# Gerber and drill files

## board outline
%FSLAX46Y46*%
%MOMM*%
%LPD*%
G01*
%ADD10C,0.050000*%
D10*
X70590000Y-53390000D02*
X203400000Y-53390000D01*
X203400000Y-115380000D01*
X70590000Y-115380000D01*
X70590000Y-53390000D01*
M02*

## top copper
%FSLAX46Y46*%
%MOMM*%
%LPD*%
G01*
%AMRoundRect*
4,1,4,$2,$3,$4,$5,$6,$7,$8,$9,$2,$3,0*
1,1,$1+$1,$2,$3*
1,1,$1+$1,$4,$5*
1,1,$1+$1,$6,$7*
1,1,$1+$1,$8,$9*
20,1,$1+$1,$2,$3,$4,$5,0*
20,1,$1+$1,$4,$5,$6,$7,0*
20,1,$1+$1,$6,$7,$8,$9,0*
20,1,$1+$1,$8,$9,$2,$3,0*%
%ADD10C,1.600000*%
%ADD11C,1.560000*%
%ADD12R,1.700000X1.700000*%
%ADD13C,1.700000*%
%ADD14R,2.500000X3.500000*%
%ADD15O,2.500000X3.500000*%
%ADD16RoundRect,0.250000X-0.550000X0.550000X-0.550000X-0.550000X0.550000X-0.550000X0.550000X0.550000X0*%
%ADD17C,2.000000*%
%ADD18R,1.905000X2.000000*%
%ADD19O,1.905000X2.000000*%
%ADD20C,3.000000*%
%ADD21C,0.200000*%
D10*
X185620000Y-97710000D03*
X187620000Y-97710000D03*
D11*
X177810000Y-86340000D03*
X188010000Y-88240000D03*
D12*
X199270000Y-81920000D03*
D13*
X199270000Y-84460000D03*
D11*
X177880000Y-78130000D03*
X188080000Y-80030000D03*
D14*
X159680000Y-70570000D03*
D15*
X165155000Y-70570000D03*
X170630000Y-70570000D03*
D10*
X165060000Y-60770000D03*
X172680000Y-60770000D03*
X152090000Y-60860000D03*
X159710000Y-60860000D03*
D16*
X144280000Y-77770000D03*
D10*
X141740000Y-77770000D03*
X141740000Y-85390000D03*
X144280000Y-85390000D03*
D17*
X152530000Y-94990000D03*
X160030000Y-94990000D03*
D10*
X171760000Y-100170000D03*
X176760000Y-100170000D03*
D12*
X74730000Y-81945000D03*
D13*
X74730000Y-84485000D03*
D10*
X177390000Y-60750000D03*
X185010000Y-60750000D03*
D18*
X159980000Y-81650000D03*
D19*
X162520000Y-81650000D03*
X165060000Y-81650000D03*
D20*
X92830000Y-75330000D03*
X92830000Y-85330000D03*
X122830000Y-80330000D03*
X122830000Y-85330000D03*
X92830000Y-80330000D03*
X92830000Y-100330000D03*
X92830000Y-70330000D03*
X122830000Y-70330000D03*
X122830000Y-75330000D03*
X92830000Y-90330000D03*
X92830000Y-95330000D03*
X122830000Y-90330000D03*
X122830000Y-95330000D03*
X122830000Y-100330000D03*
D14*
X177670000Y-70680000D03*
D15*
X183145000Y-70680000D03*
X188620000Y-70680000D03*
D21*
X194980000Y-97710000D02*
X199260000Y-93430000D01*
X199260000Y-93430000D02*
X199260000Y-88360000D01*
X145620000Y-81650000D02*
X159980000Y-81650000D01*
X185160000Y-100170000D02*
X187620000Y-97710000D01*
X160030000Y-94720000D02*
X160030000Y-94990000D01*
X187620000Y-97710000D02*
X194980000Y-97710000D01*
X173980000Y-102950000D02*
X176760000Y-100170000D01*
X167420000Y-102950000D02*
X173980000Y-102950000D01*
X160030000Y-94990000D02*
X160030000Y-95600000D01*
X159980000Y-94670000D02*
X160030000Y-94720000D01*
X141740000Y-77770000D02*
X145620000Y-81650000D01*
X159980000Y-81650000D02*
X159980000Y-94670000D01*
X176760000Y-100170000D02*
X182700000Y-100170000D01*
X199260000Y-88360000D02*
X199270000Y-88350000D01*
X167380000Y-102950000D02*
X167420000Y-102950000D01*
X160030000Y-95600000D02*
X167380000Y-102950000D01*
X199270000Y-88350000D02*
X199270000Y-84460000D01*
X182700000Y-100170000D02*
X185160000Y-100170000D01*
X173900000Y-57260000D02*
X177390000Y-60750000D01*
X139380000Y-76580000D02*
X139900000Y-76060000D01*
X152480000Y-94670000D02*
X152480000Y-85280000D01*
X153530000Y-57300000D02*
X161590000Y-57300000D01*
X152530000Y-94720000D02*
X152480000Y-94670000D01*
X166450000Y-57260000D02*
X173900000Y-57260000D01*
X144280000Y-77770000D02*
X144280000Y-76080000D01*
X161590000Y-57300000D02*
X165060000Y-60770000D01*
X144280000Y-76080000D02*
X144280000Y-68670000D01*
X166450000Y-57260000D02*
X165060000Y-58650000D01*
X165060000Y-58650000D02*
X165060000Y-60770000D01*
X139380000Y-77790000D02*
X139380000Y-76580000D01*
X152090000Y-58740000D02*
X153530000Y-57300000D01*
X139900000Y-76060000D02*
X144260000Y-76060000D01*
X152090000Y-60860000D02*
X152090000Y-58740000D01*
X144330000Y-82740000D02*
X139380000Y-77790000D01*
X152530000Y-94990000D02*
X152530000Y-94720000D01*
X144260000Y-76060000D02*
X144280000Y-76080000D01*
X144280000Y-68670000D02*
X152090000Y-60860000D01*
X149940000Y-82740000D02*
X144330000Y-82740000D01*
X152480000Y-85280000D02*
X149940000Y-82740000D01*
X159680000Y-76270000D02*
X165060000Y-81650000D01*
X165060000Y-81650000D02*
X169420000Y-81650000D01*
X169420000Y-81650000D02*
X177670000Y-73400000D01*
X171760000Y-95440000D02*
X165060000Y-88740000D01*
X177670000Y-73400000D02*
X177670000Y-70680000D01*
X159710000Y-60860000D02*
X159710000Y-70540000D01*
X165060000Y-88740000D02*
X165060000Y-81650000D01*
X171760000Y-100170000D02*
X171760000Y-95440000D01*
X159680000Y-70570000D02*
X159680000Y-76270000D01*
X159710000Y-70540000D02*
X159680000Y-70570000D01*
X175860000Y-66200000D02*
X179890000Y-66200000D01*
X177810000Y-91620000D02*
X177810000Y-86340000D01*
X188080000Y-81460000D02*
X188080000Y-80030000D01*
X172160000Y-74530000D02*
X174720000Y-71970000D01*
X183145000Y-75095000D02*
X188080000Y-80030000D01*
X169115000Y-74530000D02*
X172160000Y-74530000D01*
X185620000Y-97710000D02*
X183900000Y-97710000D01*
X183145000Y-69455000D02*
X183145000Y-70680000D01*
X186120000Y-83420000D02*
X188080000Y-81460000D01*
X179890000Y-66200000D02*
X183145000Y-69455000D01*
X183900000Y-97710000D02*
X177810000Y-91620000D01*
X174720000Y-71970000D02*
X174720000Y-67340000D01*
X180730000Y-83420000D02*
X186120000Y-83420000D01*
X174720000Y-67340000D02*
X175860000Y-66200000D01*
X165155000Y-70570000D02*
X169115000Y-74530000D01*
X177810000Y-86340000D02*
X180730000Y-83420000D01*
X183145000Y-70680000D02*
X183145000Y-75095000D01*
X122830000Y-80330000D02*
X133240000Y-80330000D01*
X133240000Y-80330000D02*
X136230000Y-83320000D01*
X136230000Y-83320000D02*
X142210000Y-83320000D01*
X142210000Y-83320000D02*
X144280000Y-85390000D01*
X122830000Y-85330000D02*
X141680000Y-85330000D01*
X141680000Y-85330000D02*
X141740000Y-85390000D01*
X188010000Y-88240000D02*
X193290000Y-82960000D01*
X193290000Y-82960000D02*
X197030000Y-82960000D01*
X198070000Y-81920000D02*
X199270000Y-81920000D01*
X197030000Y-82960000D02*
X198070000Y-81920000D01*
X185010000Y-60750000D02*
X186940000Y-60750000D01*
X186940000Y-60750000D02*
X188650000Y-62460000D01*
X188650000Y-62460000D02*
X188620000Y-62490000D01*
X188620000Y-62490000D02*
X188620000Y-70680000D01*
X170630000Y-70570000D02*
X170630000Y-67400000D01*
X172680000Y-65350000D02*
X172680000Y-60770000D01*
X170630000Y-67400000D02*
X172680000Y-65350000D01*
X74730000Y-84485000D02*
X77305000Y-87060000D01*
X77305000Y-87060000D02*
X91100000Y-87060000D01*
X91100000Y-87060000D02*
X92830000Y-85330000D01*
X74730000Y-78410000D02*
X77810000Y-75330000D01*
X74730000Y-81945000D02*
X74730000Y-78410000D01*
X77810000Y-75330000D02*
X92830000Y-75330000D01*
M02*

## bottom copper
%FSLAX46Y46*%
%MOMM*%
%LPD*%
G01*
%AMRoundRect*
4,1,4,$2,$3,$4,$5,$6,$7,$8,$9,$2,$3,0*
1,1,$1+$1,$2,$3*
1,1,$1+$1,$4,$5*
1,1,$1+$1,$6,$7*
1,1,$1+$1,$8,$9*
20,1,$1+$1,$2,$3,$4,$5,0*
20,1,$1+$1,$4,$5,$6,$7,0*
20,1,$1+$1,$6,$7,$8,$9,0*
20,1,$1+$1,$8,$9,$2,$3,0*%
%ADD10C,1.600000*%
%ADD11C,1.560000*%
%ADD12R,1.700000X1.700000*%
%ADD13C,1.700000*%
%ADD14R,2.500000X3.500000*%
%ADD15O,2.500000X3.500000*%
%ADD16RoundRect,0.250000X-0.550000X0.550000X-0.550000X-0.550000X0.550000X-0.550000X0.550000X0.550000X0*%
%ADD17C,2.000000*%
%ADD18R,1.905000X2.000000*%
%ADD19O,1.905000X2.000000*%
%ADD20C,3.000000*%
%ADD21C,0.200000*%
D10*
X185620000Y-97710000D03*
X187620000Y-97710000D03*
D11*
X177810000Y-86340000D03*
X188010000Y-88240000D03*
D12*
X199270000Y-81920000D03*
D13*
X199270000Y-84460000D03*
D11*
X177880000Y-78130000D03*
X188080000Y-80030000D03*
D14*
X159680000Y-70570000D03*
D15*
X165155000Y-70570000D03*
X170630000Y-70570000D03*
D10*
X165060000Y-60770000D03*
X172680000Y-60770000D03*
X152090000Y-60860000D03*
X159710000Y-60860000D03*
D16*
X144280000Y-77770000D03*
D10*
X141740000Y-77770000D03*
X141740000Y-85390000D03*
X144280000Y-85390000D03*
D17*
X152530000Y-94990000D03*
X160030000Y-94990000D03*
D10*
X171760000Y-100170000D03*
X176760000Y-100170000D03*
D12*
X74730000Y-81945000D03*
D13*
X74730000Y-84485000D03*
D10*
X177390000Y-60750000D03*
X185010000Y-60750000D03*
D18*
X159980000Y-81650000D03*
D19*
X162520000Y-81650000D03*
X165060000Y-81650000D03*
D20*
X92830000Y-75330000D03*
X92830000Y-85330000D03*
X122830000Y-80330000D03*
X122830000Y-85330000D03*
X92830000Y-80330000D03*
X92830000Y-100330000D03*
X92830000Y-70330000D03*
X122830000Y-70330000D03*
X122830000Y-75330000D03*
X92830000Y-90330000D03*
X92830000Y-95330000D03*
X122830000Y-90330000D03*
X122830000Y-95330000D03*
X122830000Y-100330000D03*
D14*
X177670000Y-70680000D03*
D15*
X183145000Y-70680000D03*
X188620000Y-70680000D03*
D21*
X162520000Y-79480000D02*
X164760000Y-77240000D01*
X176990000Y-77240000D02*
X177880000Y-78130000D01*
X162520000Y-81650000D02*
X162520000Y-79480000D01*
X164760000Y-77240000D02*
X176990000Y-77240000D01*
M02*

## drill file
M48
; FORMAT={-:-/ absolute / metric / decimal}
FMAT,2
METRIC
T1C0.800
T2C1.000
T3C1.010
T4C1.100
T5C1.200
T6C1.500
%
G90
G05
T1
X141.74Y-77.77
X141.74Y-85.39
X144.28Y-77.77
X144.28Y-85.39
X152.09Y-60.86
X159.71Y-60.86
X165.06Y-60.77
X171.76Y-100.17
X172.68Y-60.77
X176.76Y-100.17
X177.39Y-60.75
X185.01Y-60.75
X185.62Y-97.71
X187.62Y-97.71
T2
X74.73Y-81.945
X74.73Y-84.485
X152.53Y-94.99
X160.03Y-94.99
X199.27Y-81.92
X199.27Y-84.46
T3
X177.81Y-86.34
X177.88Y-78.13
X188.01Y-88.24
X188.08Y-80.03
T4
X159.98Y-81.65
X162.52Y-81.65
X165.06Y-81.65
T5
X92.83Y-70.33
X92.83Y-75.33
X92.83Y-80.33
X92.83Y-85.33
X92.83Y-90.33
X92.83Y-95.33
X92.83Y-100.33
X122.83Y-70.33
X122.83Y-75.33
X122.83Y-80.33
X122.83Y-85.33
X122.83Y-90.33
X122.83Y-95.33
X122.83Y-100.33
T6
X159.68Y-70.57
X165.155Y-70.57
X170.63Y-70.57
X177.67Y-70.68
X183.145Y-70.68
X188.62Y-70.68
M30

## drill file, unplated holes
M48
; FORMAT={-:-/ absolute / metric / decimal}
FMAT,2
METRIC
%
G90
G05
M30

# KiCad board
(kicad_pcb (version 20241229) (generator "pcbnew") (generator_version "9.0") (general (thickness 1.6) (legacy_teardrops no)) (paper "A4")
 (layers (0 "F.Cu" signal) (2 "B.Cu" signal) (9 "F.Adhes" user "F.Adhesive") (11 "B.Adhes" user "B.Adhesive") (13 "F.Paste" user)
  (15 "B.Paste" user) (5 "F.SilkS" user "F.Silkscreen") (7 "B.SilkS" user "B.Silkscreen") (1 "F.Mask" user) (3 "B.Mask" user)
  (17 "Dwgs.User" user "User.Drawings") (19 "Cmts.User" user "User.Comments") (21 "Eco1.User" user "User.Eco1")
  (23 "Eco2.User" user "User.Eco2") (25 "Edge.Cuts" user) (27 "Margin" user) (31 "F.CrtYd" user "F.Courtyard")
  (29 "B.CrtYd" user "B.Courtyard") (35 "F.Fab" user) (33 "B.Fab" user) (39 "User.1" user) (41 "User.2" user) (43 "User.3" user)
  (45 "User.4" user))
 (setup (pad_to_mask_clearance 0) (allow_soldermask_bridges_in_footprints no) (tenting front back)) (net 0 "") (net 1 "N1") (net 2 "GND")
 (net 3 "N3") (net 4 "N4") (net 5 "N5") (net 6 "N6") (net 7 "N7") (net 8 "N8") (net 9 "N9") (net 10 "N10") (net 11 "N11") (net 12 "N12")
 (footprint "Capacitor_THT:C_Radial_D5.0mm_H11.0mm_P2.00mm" (layer "F.Cu") (at 185.62 97.71)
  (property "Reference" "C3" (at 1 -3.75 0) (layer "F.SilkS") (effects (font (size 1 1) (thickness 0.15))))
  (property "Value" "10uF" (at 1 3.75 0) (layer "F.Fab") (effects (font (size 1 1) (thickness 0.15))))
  (pad "1" thru_hole circle (at 0 0) (size 1.6 1.6) (drill 0.8) (layers "*.Cu" "*.Mask") (remove_unused_layers no) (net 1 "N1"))
  (pad "2" thru_hole circle (at 2 0) (size 1.6 1.6) (drill 0.8) (layers "*.Cu" "*.Mask") (remove_unused_layers no) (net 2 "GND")))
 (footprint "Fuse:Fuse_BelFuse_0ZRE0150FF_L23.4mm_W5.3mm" (layer "F.Cu") (at 177.81 86.34)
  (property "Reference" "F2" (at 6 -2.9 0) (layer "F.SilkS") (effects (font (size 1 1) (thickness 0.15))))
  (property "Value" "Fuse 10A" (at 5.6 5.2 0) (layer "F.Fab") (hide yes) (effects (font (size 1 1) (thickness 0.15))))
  (pad "1" thru_hole circle (at 0 0) (size 1.56 1.56) (drill 1.01) (layers "*.Cu" "*.Mask") (remove_unused_layers no) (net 1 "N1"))
  (pad "2" thru_hole circle (at 10.2 1.9) (size 1.56 1.56) (drill 1.01) (layers "*.Cu" "*.Mask") (remove_unused_layers no) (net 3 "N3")))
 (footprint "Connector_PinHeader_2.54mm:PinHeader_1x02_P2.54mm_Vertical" (layer "F.Cu") (at 199.27 81.92)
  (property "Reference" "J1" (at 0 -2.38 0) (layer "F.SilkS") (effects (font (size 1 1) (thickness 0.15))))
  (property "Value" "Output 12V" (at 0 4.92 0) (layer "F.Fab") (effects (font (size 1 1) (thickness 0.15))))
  (pad "1" thru_hole rect (at 0 0) (size 1.7 1.7) (drill 1) (layers "*.Cu" "*.Mask") (remove_unused_layers no) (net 3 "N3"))
  (pad "2" thru_hole circle (at 0 2.54) (size 1.7 1.7) (drill 1) (layers "*.Cu" "*.Mask") (remove_unused_layers no) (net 2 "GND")))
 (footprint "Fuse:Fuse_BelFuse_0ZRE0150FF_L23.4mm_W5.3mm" (layer "F.Cu") (at 177.88 78.13)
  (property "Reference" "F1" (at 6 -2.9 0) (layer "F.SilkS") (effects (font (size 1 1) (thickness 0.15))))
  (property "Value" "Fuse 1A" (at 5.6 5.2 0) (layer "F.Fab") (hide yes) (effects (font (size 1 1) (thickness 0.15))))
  (pad "1" thru_hole circle (at 0 0) (size 1.56 1.56) (drill 1.01) (layers "*.Cu" "*.Mask") (remove_unused_layers no) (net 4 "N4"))
  (pad "2" thru_hole circle (at 10.2 1.9) (size 1.56 1.56) (drill 1.01) (layers "*.Cu" "*.Mask") (remove_unused_layers no) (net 1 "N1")))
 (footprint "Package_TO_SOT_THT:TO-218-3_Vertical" (layer "F.Cu") (at 159.68 70.57)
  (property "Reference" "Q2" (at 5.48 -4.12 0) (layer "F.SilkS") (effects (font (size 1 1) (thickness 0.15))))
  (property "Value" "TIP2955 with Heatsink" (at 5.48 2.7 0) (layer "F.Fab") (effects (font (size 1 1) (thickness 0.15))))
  (pad "1" thru_hole rect (at 0 0) (size 2.5 3.5) (drill 1.5) (layers "*.Cu" "*.Mask") (remove_unused_layers no) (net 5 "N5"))
  (pad "2" thru_hole oval (at 5.475 0) (size 2.5 3.5) (drill 1.5) (layers "*.Cu" "*.Mask") (remove_unused_layers no) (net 1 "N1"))
  (pad "3" thru_hole oval (at 10.95 0) (size 2.5 3.5) (drill 1.5) (layers "*.Cu" "*.Mask") (remove_unused_layers no) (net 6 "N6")))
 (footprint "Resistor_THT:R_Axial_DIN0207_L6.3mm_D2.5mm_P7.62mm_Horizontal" (layer "F.Cu") (at 165.06 60.77)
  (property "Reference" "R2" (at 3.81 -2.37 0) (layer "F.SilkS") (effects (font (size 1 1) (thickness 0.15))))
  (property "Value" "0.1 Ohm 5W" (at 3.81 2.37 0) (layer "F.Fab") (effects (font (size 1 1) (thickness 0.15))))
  (pad "1" thru_hole circle (at 0 0) (size 1.6 1.6) (drill 0.8) (layers "*.Cu" "*.Mask") (remove_unused_layers no) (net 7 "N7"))
  (pad "2" thru_hole circle (at 7.62 0) (size 1.6 1.6) (drill 0.8) (layers "*.Cu" "*.Mask") (remove_unused_layers no) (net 6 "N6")))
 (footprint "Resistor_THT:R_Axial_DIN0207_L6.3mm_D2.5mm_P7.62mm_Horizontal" (layer "F.Cu") (at 152.09 60.86)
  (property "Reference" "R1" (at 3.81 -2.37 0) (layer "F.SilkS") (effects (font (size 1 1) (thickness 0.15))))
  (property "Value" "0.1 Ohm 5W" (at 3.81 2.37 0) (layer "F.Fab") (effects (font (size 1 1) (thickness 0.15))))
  (pad "1" thru_hole circle (at 0 0) (size 1.6 1.6) (drill 0.8) (layers "*.Cu" "*.Mask") (remove_unused_layers no) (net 7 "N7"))
  (pad "2" thru_hole circle (at 7.62 0) (size 1.6 1.6) (drill 0.8) (layers "*.Cu" "*.Mask") (remove_unused_layers no) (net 5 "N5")))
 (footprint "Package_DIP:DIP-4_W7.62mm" (layer "F.Cu") (at 144.28 77.77 -90)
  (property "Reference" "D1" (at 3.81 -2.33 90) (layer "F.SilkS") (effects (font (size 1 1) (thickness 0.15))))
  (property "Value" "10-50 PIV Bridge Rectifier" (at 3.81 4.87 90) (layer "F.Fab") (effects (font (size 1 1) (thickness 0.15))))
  (pad "1" thru_hole roundrect (at 0 0 270) (size 1.6 1.6) (drill 0.8) (layers "*.Cu" "*.Mask") (remove_unused_layers no)
   (roundrect_rratio 0.15625) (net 7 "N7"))
  (pad "2" thru_hole circle (at 0 2.54 270) (size 1.6 1.6) (drill 0.8) (layers "*.Cu" "*.Mask") (remove_unused_layers no) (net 2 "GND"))
  (pad "3" thru_hole circle (at 7.62 2.54 270) (size 1.6 1.6) (drill 0.8) (layers "*.Cu" "*.Mask") (remove_unused_layers no) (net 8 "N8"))
  (pad "4" thru_hole circle (at 7.62 0 270) (size 1.6 1.6) (drill 0.8) (layers "*.Cu" "*.Mask") (remove_unused_layers no) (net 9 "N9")))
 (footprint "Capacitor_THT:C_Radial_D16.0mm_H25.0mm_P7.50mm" (layer "F.Cu") (at 152.53 94.99)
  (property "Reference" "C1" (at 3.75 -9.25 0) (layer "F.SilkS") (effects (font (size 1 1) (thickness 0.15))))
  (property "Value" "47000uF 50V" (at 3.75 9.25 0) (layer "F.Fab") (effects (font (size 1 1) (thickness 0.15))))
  (pad "1" thru_hole circle (at 0 0) (size 2 2) (drill 1) (layers "*.Cu" "*.Mask") (remove_unused_layers no) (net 7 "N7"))
  (pad "2" thru_hole circle (at 7.5 0) (size 2 2) (drill 1) (layers "*.Cu" "*.Mask") (remove_unused_layers no) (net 2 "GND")))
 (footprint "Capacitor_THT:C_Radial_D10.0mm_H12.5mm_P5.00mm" (layer "F.Cu") (at 171.76 100.17)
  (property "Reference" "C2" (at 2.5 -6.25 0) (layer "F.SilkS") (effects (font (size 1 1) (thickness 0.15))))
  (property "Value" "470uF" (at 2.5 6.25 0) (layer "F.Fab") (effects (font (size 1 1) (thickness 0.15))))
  (pad "1" thru_hole circle (at 0 0) (size 1.6 1.6) (drill 0.8) (layers "*.Cu" "*.Mask") (remove_unused_layers no) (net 5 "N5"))
  (pad "2" thru_hole circle (at 5 0) (size 1.6 1.6) (drill 0.8) (layers "*.Cu" "*.Mask") (remove_unused_layers no) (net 2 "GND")))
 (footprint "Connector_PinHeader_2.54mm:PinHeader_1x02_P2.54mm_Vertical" (layer "F.Cu") (at 74.73 81.945)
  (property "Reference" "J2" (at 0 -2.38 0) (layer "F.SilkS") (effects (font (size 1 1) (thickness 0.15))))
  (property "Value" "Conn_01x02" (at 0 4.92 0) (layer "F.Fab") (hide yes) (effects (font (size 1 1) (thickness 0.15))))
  (pad "1" thru_hole rect (at 0 0) (size 1.7 1.7) (drill 1) (layers "*.Cu" "*.Mask") (remove_unused_layers no) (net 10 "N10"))
  (pad "2" thru_hole circle (at 0 2.54) (size 1.7 1.7) (drill 1) (layers "*.Cu" "*.Mask") (remove_unused_layers no) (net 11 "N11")))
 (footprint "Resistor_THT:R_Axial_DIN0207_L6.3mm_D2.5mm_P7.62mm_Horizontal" (layer "F.Cu") (at 177.39 60.75)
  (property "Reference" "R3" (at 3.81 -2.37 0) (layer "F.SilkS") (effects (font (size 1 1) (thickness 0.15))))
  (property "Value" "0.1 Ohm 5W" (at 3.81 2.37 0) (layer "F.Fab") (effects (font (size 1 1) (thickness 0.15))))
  (pad "1" thru_hole circle (at 0 0) (size 1.6 1.6) (drill 0.8) (layers "*.Cu" "*.Mask") (remove_unused_layers no) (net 7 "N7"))
  (pad "2" thru_hole circle (at 7.62 0) (size 1.6 1.6) (drill 0.8) (layers "*.Cu" "*.Mask") (remove_unused_layers no) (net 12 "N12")))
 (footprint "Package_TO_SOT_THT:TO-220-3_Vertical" (layer "F.Cu") (at 159.98 81.65)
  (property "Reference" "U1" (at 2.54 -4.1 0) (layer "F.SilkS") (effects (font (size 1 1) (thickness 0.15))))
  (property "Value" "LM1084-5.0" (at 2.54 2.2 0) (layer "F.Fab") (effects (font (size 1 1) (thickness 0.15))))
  (pad "1" thru_hole rect (at 0 0) (size 1.905 2) (drill 1.1) (layers "*.Cu" "*.Mask") (remove_unused_layers no) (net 2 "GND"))
  (pad "2" thru_hole oval (at 2.54 0) (size 1.905 2) (drill 1.1) (layers "*.Cu" "*.Mask") (remove_unused_layers no) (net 4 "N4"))
  (pad "3" thru_hole oval (at 5.08 0) (size 1.905 2) (drill 1.1) (layers "*.Cu" "*.Mask") (remove_unused_layers no) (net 5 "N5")))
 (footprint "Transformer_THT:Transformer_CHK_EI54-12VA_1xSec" (layer "F.Cu") (at 92.83 100.33)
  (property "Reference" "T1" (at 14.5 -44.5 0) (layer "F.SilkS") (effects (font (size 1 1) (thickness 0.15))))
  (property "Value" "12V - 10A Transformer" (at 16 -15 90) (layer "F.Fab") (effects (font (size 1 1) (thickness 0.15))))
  (pad "1" thru_hole circle (at 0 -25) (size 3 3) (drill 1.2) (layers "*.Cu" "*.Mask") (remove_unused_layers no) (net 10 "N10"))
  (pad "2" thru_hole circle (at 0 -15) (size 3 3) (drill 1.2) (layers "*.Cu" "*.Mask") (remove_unused_layers no) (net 11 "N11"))
  (pad "3" thru_hole circle (at 30 -20) (size 3 3) (drill 1.2) (layers "*.Cu" "*.Mask") (remove_unused_layers no) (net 9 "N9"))
  (pad "4" thru_hole circle (at 30 -15) (size 3 3) (drill 1.2) (layers "*.Cu" "*.Mask") (remove_unused_layers no) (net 8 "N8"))
  (pad "5" thru_hole circle (at 0 -20) (size 3 3) (drill 1.2) (layers "*.Cu" "*.Mask") (remove_unused_layers no))
  (pad "6" thru_hole circle (at 0 0) (size 3 3) (drill 1.2) (layers "*.Cu" "*.Mask") (remove_unused_layers no))
  (pad "7" thru_hole circle (at 0 -30) (size 3 3) (drill 1.2) (layers "*.Cu" "*.Mask") (remove_unused_layers no))
  (pad "8" thru_hole circle (at 30 -30) (size 3 3) (drill 1.2) (layers "*.Cu" "*.Mask") (remove_unused_layers no))
  (pad "9" thru_hole circle (at 30 -25) (size 3 3) (drill 1.2) (layers "*.Cu" "*.Mask") (remove_unused_layers no))
  (pad "10" thru_hole circle (at 0 -10) (size 3 3) (drill 1.2) (layers "*.Cu" "*.Mask") (remove_unused_layers no))
  (pad "11" thru_hole circle (at 0 -5) (size 3 3) (drill 1.2) (layers "*.Cu" "*.Mask") (remove_unused_layers no))
  (pad "12" thru_hole circle (at 30 -10) (size 3 3) (drill 1.2) (layers "*.Cu" "*.Mask") (remove_unused_layers no))
  (pad "13" thru_hole circle (at 30 -5) (size 3 3) (drill 1.2) (layers "*.Cu" "*.Mask") (remove_unused_layers no))
  (pad "14" thru_hole circle (at 30 0) (size 3 3) (drill 1.2) (layers "*.Cu" "*.Mask") (remove_unused_layers no)))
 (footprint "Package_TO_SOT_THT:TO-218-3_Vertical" (layer "F.Cu") (at 177.67 70.68)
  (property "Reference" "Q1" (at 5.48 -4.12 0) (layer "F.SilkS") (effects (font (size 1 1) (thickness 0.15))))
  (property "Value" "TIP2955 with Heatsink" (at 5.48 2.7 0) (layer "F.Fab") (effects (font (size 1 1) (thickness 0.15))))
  (pad "1" thru_hole rect (at 0 0) (size 2.5 3.5) (drill 1.5) (layers "*.Cu" "*.Mask") (remove_unused_layers no) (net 5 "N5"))
  (pad "2" thru_hole oval (at 5.475 0) (size 2.5 3.5) (drill 1.5) (layers "*.Cu" "*.Mask") (remove_unused_layers no) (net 1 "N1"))
  (pad "3" thru_hole oval (at 10.95 0) (size 2.5 3.5) (drill 1.5) (layers "*.Cu" "*.Mask") (remove_unused_layers no) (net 12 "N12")))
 (gr_rect (start 70.59 53.39) (end 203.4 115.38) (stroke (width 0.05) (type default)) (fill no) (layer "Edge.Cuts"))
 (segment (start 194.98 97.71) (end 199.26 93.43) (width 0.2) (layer "F.Cu") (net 2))
 (segment (start 199.26 93.43) (end 199.26 88.36) (width 0.2) (layer "F.Cu") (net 2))
 (segment (start 145.62 81.65) (end 159.98 81.65) (width 0.2) (layer "F.Cu") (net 2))
 (segment (start 185.16 100.17) (end 187.62 97.71) (width 0.2) (layer "F.Cu") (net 2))
 (segment (start 160.03 94.72) (end 160.03 94.99) (width 0.2) (layer "F.Cu") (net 2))
 (segment (start 187.62 97.71) (end 194.98 97.71) (width 0.2) (layer "F.Cu") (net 2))
 (segment (start 173.98 102.95) (end 176.76 100.17) (width 0.2) (layer "F.Cu") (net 2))
 (segment (start 167.42 102.95) (end 173.98 102.95) (width 0.2) (layer "F.Cu") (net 2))
 (segment (start 160.03 94.99) (end 160.03 95.6) (width 0.2) (layer "F.Cu") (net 2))
 (segment (start 159.98 94.67) (end 160.03 94.72) (width 0.2) (layer "F.Cu") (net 2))
 (segment (start 141.74 77.77) (end 145.62 81.65) (width 0.2) (layer "F.Cu") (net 2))
 (segment (start 159.98 81.65) (end 159.98 94.67) (width 0.2) (layer "F.Cu") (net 2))
 (segment (start 176.76 100.17) (end 182.7 100.17) (width 0.2) (layer "F.Cu") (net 2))
 (segment (start 199.26 88.36) (end 199.27 88.35) (width 0.2) (layer "F.Cu") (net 2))
 (segment (start 167.38 102.95) (end 167.42 102.95) (width 0.2) (layer "F.Cu") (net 2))
 (segment (start 160.03 95.6) (end 167.38 102.95) (width 0.2) (layer "F.Cu") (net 2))
 (segment (start 199.27 88.35) (end 199.27 84.46) (width 0.2) (layer "F.Cu") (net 2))
 (segment (start 182.7 100.17) (end 185.16 100.17) (width 0.2) (layer "F.Cu") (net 2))
 (segment (start 173.9 57.26) (end 177.39 60.75) (width 0.2) (layer "F.Cu") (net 7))
 (segment (start 139.38 76.58) (end 139.9 76.06) (width 0.2) (layer "F.Cu") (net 7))
 (segment (start 152.48 94.67) (end 152.48 85.28) (width 0.2) (layer "F.Cu") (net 7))
 (segment (start 153.53 57.3) (end 161.59 57.3) (width 0.2) (layer "F.Cu") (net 7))
 (segment (start 152.53 94.72) (end 152.48 94.67) (width 0.2) (layer "F.Cu") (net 7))
 (segment (start 166.45 57.26) (end 173.9 57.26) (width 0.2) (layer "F.Cu") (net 7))
 (segment (start 144.28 77.77) (end 144.28 76.08) (width 0.2) (layer "F.Cu") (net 7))
 (segment (start 161.59 57.3) (end 165.06 60.77) (width 0.2) (layer "F.Cu") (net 7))
 (segment (start 144.28 76.08) (end 144.28 68.67) (width 0.2) (layer "F.Cu") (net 7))
 (segment (start 166.45 57.26) (end 165.06 58.65) (width 0.2) (layer "F.Cu") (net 7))
 (segment (start 165.06 58.65) (end 165.06 60.77) (width 0.2) (layer "F.Cu") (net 7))
 (segment (start 139.38 77.79) (end 139.38 76.58) (width 0.2) (layer "F.Cu") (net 7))
 (segment (start 152.09 58.74) (end 153.53 57.3) (width 0.2) (layer "F.Cu") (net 7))
 (segment (start 139.9 76.06) (end 144.26 76.06) (width 0.2) (layer "F.Cu") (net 7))
 (segment (start 152.09 60.86) (end 152.09 58.74) (width 0.2) (layer "F.Cu") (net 7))
 (segment (start 144.33 82.74) (end 139.38 77.79) (width 0.2) (layer "F.Cu") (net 7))
 (segment (start 152.53 94.99) (end 152.53 94.72) (width 0.2) (layer "F.Cu") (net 7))
 (segment (start 144.26 76.06) (end 144.28 76.08) (width 0.2) (layer "F.Cu") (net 7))
 (segment (start 144.28 68.67) (end 152.09 60.86) (width 0.2) (layer "F.Cu") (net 7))
 (segment (start 149.94 82.74) (end 144.33 82.74) (width 0.2) (layer "F.Cu") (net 7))
 (segment (start 152.48 85.28) (end 149.94 82.74) (width 0.2) (layer "F.Cu") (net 7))
 (segment (start 159.68 76.27) (end 165.06 81.65) (width 0.2) (layer "F.Cu") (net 5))
 (segment (start 165.06 81.65) (end 169.42 81.65) (width 0.2) (layer "F.Cu") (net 5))
 (segment (start 169.42 81.65) (end 177.67 73.4) (width 0.2) (layer "F.Cu") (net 5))
 (segment (start 171.76 95.44) (end 165.06 88.74) (width 0.2) (layer "F.Cu") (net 5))
 (segment (start 177.67 73.4) (end 177.67 70.68) (width 0.2) (layer "F.Cu") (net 5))
 (segment (start 159.71 60.86) (end 159.71 70.54) (width 0.2) (layer "F.Cu") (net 5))
 (segment (start 165.06 88.74) (end 165.06 81.65) (width 0.2) (layer "F.Cu") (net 5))
 (segment (start 171.76 100.17) (end 171.76 95.44) (width 0.2) (layer "F.Cu") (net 5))
 (segment (start 159.68 70.57) (end 159.68 76.27) (width 0.2) (layer "F.Cu") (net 5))
 (segment (start 159.71 70.54) (end 159.68 70.57) (width 0.2) (layer "F.Cu") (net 5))
 (segment (start 175.86 66.2) (end 179.89 66.2) (width 0.2) (layer "F.Cu") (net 1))
 (segment (start 177.81 91.62) (end 177.81 86.34) (width 0.2) (layer "F.Cu") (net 1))
 (segment (start 188.08 81.46) (end 188.08 80.03) (width 0.2) (layer "F.Cu") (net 1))
 (segment (start 172.16 74.53) (end 174.72 71.97) (width 0.2) (layer "F.Cu") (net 1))
 (segment (start 183.145 75.095) (end 188.08 80.03) (width 0.2) (layer "F.Cu") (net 1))
 (segment (start 169.115 74.53) (end 172.16 74.53) (width 0.2) (layer "F.Cu") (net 1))
 (segment (start 185.62 97.71) (end 183.9 97.71) (width 0.2) (layer "F.Cu") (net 1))
 (segment (start 183.145 69.455) (end 183.145 70.68) (width 0.2) (layer "F.Cu") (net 1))
 (segment (start 186.12 83.42) (end 188.08 81.46) (width 0.2) (layer "F.Cu") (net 1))
 (segment (start 179.89 66.2) (end 183.145 69.455) (width 0.2) (layer "F.Cu") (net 1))
 (segment (start 183.9 97.71) (end 177.81 91.62) (width 0.2) (layer "F.Cu") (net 1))
 (segment (start 174.72 71.97) (end 174.72 67.34) (width 0.2) (layer "F.Cu") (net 1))
 (segment (start 180.73 83.42) (end 186.12 83.42) (width 0.2) (layer "F.Cu") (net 1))
 (segment (start 174.72 67.34) (end 175.86 66.2) (width 0.2) (layer "F.Cu") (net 1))
 (segment (start 165.155 70.57) (end 169.115 74.53) (width 0.2) (layer "F.Cu") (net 1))
 (segment (start 177.81 86.34) (end 180.73 83.42) (width 0.2) (layer "F.Cu") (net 1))
 (segment (start 183.145 70.68) (end 183.145 75.095) (width 0.2) (layer "F.Cu") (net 1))
 (segment (start 122.83 80.33) (end 133.24 80.33) (width 0.2) (layer "F.Cu") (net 9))
 (segment (start 133.24 80.33) (end 136.23 83.32) (width 0.2) (layer "F.Cu") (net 9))
 (segment (start 136.23 83.32) (end 142.21 83.32) (width 0.2) (layer "F.Cu") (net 9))
 (segment (start 142.21 83.32) (end 144.28 85.39) (width 0.2) (layer "F.Cu") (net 9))
 (segment (start 122.83 85.33) (end 141.68 85.33) (width 0.2) (layer "F.Cu") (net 8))
 (segment (start 141.68 85.33) (end 141.74 85.39) (width 0.2) (layer "F.Cu") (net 8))
 (segment (start 162.52 79.48) (end 164.76 77.24) (width 0.2) (layer "B.Cu") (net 4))
 (segment (start 176.99 77.24) (end 177.88 78.13) (width 0.2) (layer "B.Cu") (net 4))
 (segment (start 162.52 81.65) (end 162.52 79.48) (width 0.2) (layer "B.Cu") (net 4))
 (segment (start 164.76 77.24) (end 176.99 77.24) (width 0.2) (layer "B.Cu") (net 4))
 (segment (start 188.01 88.24) (end 193.29 82.96) (width 0.2) (layer "F.Cu") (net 3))
 (segment (start 193.29 82.96) (end 197.03 82.96) (width 0.2) (layer "F.Cu") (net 3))
 (segment (start 198.07 81.92) (end 199.27 81.92) (width 0.2) (layer "F.Cu") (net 3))
 (segment (start 197.03 82.96) (end 198.07 81.92) (width 0.2) (layer "F.Cu") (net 3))
 (segment (start 185.01 60.75) (end 186.94 60.75) (width 0.2) (layer "F.Cu") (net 12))
 (segment (start 186.94 60.75) (end 188.65 62.46) (width 0.2) (layer "F.Cu") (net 12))
 (segment (start 188.65 62.46) (end 188.62 62.49) (width 0.2) (layer "F.Cu") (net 12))
 (segment (start 188.62 62.49) (end 188.62 70.68) (width 0.2) (layer "F.Cu") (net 12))
 (segment (start 170.63 70.57) (end 170.63 67.4) (width 0.2) (layer "F.Cu") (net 6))
 (segment (start 172.68 65.35) (end 172.68 60.77) (width 0.2) (layer "F.Cu") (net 6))
 (segment (start 170.63 67.4) (end 172.68 65.35) (width 0.2) (layer "F.Cu") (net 6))
 (segment (start 74.73 84.485) (end 77.305 87.06) (width 0.2) (layer "F.Cu") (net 11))
 (segment (start 77.305 87.06) (end 91.1 87.06) (width 0.2) (layer "F.Cu") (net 11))
 (segment (start 91.1 87.06) (end 92.83 85.33) (width 0.2) (layer "F.Cu") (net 11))
 (segment (start 74.73 78.41) (end 77.81 75.33) (width 0.2) (layer "F.Cu") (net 10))
 (segment (start 74.73 81.945) (end 74.73 78.41) (width 0.2) (layer "F.Cu") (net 10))
 (segment (start 77.81 75.33) (end 92.83 75.33) (width 0.2) (layer "F.Cu") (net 10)))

